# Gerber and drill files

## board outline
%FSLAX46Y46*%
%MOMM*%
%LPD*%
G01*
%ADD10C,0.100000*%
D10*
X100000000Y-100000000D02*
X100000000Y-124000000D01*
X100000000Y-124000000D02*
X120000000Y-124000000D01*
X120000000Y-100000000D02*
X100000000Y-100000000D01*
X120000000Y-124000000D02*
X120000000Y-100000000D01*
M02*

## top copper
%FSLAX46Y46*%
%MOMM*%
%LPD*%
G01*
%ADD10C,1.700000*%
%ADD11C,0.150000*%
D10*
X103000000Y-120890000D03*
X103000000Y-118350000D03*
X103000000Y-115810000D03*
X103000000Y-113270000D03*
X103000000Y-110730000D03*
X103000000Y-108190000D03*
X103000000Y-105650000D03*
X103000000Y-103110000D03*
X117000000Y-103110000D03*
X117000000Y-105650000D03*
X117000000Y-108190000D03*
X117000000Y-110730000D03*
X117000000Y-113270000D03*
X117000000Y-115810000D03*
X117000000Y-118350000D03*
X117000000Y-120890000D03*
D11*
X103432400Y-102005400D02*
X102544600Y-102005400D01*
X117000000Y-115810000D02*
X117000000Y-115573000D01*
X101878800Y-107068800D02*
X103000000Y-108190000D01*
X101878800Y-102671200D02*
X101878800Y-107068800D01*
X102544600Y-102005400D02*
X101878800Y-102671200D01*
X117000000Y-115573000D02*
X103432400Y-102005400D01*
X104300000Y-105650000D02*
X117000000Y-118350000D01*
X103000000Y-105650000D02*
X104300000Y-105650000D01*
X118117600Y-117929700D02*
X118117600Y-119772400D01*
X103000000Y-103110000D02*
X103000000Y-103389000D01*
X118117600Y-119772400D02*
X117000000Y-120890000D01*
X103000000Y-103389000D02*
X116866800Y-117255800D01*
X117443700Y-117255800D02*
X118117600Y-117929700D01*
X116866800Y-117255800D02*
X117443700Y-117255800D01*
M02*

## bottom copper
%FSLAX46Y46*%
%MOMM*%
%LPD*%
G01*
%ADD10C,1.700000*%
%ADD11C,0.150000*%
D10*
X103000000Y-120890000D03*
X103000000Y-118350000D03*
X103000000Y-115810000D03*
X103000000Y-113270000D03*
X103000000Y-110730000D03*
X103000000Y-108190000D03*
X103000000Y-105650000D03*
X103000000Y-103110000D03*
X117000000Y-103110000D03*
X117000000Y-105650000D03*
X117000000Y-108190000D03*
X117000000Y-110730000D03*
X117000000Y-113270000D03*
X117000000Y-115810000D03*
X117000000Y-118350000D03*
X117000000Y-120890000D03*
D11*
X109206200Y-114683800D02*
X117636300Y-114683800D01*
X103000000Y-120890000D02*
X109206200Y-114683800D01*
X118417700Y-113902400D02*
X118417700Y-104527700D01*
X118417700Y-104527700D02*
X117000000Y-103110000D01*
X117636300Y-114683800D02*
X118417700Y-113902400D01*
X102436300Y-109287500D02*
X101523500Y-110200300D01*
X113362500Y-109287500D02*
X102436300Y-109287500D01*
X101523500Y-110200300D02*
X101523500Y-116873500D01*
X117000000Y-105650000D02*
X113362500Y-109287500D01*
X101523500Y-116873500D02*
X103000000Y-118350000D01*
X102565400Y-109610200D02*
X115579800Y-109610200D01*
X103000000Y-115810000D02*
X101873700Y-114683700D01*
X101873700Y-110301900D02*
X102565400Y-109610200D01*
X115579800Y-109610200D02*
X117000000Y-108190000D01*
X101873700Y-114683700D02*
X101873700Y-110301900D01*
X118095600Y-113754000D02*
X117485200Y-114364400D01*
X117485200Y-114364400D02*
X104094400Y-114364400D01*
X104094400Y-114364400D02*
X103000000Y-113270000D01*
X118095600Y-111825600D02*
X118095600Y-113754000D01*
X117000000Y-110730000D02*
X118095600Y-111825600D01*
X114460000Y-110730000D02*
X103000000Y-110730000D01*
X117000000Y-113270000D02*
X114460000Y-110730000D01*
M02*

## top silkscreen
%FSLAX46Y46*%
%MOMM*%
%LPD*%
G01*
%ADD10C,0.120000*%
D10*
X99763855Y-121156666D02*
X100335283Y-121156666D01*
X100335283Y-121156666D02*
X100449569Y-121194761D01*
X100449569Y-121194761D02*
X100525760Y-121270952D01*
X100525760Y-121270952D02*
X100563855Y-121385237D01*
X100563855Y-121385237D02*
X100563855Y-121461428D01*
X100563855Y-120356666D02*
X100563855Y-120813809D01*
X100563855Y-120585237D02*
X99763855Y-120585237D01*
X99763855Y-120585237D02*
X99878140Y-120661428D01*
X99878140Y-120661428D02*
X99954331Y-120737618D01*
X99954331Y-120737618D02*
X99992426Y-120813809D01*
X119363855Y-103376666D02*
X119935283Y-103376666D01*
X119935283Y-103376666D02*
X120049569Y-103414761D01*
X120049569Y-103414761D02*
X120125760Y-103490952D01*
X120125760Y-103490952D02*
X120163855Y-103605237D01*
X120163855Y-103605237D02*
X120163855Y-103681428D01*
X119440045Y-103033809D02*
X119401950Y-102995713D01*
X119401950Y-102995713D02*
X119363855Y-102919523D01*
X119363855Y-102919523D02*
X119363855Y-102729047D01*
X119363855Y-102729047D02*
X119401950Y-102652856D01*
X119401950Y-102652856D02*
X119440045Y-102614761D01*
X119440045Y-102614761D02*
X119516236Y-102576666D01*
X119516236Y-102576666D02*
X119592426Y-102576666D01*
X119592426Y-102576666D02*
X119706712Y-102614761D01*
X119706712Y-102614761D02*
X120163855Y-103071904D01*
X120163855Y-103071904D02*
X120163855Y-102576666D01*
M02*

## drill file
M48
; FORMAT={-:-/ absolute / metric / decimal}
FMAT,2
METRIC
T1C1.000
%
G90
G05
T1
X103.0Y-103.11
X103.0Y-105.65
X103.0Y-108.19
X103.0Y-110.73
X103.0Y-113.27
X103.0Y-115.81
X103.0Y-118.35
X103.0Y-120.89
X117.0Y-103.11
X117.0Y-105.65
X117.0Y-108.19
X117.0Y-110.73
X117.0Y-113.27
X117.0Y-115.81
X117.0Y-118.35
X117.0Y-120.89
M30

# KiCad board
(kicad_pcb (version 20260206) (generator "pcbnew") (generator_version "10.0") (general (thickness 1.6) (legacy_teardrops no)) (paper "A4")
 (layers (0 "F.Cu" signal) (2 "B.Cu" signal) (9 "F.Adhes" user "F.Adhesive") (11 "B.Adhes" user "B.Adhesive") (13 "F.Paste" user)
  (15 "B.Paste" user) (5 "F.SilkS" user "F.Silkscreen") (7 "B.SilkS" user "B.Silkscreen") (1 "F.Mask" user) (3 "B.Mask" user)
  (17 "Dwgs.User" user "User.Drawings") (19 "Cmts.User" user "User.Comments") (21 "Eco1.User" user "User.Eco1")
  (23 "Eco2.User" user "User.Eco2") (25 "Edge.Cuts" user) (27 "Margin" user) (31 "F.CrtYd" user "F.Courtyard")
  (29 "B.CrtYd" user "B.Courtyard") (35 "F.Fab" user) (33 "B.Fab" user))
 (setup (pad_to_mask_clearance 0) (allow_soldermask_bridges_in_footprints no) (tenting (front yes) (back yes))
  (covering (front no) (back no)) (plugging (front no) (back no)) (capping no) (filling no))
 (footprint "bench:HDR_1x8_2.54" (layer "F.Cu") (at 103 120.89 90)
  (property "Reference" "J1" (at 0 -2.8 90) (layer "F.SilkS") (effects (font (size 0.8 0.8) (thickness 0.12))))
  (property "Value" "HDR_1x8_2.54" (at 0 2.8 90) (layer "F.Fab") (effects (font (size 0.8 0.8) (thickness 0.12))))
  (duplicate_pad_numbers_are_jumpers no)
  (pad "1" thru_hole circle (at 0 0 90) (size 1.7 1.7) (drill 1) (layers "*.Cu" "*.Mask") (remove_unused_layers no) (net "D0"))
  (pad "2" thru_hole circle (at 2.54 0 90) (size 1.7 1.7) (drill 1) (layers "*.Cu" "*.Mask") (remove_unused_layers no) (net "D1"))
  (pad "3" thru_hole circle (at 5.08 0 90) (size 1.7 1.7) (drill 1) (layers "*.Cu" "*.Mask") (remove_unused_layers no) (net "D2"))
  (pad "4" thru_hole circle (at 7.62 0 90) (size 1.7 1.7) (drill 1) (layers "*.Cu" "*.Mask") (remove_unused_layers no) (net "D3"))
  (pad "5" thru_hole circle (at 10.16 0 90) (size 1.7 1.7) (drill 1) (layers "*.Cu" "*.Mask") (remove_unused_layers no) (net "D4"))
  (pad "6" thru_hole circle (at 12.7 0 90) (size 1.7 1.7) (drill 1) (layers "*.Cu" "*.Mask") (remove_unused_layers no) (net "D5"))
  (pad "7" thru_hole circle (at 15.24 0 90) (size 1.7 1.7) (drill 1) (layers "*.Cu" "*.Mask") (remove_unused_layers no) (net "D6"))
  (pad "8" thru_hole circle (at 17.78 0 90) (size 1.7 1.7) (drill 1) (layers "*.Cu" "*.Mask") (remove_unused_layers no) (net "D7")))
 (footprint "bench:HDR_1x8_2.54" (layer "F.Cu") (at 117 103.11 -90)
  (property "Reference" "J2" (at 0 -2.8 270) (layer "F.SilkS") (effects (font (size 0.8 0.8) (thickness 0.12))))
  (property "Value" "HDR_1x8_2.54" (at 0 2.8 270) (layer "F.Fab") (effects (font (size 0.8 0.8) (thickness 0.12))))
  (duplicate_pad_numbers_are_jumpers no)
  (pad "1" thru_hole circle (at 0 0 270) (size 1.7 1.7) (drill 1) (layers "*.Cu" "*.Mask") (remove_unused_layers no) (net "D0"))
  (pad "2" thru_hole circle (at 2.54 0 270) (size 1.7 1.7) (drill 1) (layers "*.Cu" "*.Mask") (remove_unused_layers no) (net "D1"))
  (pad "3" thru_hole circle (at 5.08 0 270) (size 1.7 1.7) (drill 1) (layers "*.Cu" "*.Mask") (remove_unused_layers no) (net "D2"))
  (pad "4" thru_hole circle (at 7.62 0 270) (size 1.7 1.7) (drill 1) (layers "*.Cu" "*.Mask") (remove_unused_layers no) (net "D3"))
  (pad "5" thru_hole circle (at 10.16 0 270) (size 1.7 1.7) (drill 1) (layers "*.Cu" "*.Mask") (remove_unused_layers no) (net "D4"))
  (pad "6" thru_hole circle (at 12.7 0 270) (size 1.7 1.7) (drill 1) (layers "*.Cu" "*.Mask") (remove_unused_layers no) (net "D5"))
  (pad "7" thru_hole circle (at 15.24 0 270) (size 1.7 1.7) (drill 1) (layers "*.Cu" "*.Mask") (remove_unused_layers no) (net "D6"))
  (pad "8" thru_hole circle (at 17.78 0 270) (size 1.7 1.7) (drill 1) (layers "*.Cu" "*.Mask") (remove_unused_layers no) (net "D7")))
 (gr_line (start 100 100) (end 100 124) (stroke (width 0.1) (type solid)) (layer "Edge.Cuts"))
 (gr_line (start 100 124) (end 120 124) (stroke (width 0.1) (type solid)) (layer "Edge.Cuts"))
 (gr_line (start 120 100) (end 100 100) (stroke (width 0.1) (type solid)) (layer "Edge.Cuts"))
 (gr_line (start 120 124) (end 120 100) (stroke (width 0.1) (type solid)) (layer "Edge.Cuts"))
 (segment (start 109.2062 114.6838) (end 117.6363 114.6838) (width 0.15) (layer "B.Cu") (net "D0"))
 (segment (start 103 120.89) (end 109.2062 114.6838) (width 0.15) (layer "B.Cu") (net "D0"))
 (segment (start 118.4177 113.9024) (end 118.4177 104.5277) (width 0.15) (layer "B.Cu") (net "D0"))
 (segment (start 118.4177 104.5277) (end 117 103.11) (width 0.15) (layer "B.Cu") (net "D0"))
 (segment (start 117.6363 114.6838) (end 118.4177 113.9024) (width 0.15) (layer "B.Cu") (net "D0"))
 (segment (start 102.4363 109.2875) (end 101.5235 110.2003) (width 0.15) (layer "B.Cu") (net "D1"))
 (segment (start 113.3625 109.2875) (end 102.4363 109.2875) (width 0.15) (layer "B.Cu") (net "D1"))
 (segment (start 101.5235 110.2003) (end 101.5235 116.8735) (width 0.15) (layer "B.Cu") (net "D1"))
 (segment (start 117 105.65) (end 113.3625 109.2875) (width 0.15) (layer "B.Cu") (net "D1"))
 (segment (start 101.5235 116.8735) (end 103 118.35) (width 0.15) (layer "B.Cu") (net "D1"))
 (segment (start 102.5654 109.6102) (end 115.5798 109.6102) (width 0.15) (layer "B.Cu") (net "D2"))
 (segment (start 103 115.81) (end 101.8737 114.6837) (width 0.15) (layer "B.Cu") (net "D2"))
 (segment (start 101.8737 110.3019) (end 102.5654 109.6102) (width 0.15) (layer "B.Cu") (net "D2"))
 (segment (start 115.5798 109.6102) (end 117 108.19) (width 0.15) (layer "B.Cu") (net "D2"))
 (segment (start 101.8737 114.6837) (end 101.8737 110.3019) (width 0.15) (layer "B.Cu") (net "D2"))
 (segment (start 118.0956 113.754) (end 117.4852 114.3644) (width 0.15) (layer "B.Cu") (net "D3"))
 (segment (start 117.4852 114.3644) (end 104.0944 114.3644) (width 0.15) (layer "B.Cu") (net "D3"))
 (segment (start 104.0944 114.3644) (end 103 113.27) (width 0.15) (layer "B.Cu") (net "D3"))
 (segment (start 118.0956 111.8256) (end 118.0956 113.754) (width 0.15) (layer "B.Cu") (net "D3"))
 (segment (start 117 110.73) (end 118.0956 111.8256) (width 0.15) (layer "B.Cu") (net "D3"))
 (segment (start 114.46 110.73) (end 103 110.73) (width 0.15) (layer "B.Cu") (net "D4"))
 (segment (start 117 113.27) (end 114.46 110.73) (width 0.15) (layer "B.Cu") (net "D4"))
 (segment (start 103.4324 102.0054) (end 102.5446 102.0054) (width 0.15) (layer "F.Cu") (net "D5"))
 (segment (start 117 115.81) (end 117 115.573) (width 0.15) (layer "F.Cu") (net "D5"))
 (segment (start 101.8788 107.0688) (end 103 108.19) (width 0.15) (layer "F.Cu") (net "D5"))
 (segment (start 101.8788 102.6712) (end 101.8788 107.0688) (width 0.15) (layer "F.Cu") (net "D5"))
 (segment (start 102.5446 102.0054) (end 101.8788 102.6712) (width 0.15) (layer "F.Cu") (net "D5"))
 (segment (start 117 115.573) (end 103.4324 102.0054) (width 0.15) (layer "F.Cu") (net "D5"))
 (segment (start 104.3 105.65) (end 117 118.35) (width 0.15) (layer "F.Cu") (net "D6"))
 (segment (start 103 105.65) (end 104.3 105.65) (width 0.15) (layer "F.Cu") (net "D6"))
 (segment (start 118.1176 117.9297) (end 118.1176 119.7724) (width 0.15) (layer "F.Cu") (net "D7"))
 (segment (start 103 103.11) (end 103 103.389) (width 0.15) (layer "F.Cu") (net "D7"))
 (segment (start 118.1176 119.7724) (end 117 120.89) (width 0.15) (layer "F.Cu") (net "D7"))
 (segment (start 103 103.389) (end 116.8668 117.2558) (width 0.15) (layer "F.Cu") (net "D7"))
 (segment (start 117.4437 117.2558) (end 118.1176 117.9297) (width 0.15) (layer "F.Cu") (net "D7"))
 (segment (start 116.8668 117.2558) (end 117.4437 117.2558) (width 0.15) (layer "F.Cu") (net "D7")))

